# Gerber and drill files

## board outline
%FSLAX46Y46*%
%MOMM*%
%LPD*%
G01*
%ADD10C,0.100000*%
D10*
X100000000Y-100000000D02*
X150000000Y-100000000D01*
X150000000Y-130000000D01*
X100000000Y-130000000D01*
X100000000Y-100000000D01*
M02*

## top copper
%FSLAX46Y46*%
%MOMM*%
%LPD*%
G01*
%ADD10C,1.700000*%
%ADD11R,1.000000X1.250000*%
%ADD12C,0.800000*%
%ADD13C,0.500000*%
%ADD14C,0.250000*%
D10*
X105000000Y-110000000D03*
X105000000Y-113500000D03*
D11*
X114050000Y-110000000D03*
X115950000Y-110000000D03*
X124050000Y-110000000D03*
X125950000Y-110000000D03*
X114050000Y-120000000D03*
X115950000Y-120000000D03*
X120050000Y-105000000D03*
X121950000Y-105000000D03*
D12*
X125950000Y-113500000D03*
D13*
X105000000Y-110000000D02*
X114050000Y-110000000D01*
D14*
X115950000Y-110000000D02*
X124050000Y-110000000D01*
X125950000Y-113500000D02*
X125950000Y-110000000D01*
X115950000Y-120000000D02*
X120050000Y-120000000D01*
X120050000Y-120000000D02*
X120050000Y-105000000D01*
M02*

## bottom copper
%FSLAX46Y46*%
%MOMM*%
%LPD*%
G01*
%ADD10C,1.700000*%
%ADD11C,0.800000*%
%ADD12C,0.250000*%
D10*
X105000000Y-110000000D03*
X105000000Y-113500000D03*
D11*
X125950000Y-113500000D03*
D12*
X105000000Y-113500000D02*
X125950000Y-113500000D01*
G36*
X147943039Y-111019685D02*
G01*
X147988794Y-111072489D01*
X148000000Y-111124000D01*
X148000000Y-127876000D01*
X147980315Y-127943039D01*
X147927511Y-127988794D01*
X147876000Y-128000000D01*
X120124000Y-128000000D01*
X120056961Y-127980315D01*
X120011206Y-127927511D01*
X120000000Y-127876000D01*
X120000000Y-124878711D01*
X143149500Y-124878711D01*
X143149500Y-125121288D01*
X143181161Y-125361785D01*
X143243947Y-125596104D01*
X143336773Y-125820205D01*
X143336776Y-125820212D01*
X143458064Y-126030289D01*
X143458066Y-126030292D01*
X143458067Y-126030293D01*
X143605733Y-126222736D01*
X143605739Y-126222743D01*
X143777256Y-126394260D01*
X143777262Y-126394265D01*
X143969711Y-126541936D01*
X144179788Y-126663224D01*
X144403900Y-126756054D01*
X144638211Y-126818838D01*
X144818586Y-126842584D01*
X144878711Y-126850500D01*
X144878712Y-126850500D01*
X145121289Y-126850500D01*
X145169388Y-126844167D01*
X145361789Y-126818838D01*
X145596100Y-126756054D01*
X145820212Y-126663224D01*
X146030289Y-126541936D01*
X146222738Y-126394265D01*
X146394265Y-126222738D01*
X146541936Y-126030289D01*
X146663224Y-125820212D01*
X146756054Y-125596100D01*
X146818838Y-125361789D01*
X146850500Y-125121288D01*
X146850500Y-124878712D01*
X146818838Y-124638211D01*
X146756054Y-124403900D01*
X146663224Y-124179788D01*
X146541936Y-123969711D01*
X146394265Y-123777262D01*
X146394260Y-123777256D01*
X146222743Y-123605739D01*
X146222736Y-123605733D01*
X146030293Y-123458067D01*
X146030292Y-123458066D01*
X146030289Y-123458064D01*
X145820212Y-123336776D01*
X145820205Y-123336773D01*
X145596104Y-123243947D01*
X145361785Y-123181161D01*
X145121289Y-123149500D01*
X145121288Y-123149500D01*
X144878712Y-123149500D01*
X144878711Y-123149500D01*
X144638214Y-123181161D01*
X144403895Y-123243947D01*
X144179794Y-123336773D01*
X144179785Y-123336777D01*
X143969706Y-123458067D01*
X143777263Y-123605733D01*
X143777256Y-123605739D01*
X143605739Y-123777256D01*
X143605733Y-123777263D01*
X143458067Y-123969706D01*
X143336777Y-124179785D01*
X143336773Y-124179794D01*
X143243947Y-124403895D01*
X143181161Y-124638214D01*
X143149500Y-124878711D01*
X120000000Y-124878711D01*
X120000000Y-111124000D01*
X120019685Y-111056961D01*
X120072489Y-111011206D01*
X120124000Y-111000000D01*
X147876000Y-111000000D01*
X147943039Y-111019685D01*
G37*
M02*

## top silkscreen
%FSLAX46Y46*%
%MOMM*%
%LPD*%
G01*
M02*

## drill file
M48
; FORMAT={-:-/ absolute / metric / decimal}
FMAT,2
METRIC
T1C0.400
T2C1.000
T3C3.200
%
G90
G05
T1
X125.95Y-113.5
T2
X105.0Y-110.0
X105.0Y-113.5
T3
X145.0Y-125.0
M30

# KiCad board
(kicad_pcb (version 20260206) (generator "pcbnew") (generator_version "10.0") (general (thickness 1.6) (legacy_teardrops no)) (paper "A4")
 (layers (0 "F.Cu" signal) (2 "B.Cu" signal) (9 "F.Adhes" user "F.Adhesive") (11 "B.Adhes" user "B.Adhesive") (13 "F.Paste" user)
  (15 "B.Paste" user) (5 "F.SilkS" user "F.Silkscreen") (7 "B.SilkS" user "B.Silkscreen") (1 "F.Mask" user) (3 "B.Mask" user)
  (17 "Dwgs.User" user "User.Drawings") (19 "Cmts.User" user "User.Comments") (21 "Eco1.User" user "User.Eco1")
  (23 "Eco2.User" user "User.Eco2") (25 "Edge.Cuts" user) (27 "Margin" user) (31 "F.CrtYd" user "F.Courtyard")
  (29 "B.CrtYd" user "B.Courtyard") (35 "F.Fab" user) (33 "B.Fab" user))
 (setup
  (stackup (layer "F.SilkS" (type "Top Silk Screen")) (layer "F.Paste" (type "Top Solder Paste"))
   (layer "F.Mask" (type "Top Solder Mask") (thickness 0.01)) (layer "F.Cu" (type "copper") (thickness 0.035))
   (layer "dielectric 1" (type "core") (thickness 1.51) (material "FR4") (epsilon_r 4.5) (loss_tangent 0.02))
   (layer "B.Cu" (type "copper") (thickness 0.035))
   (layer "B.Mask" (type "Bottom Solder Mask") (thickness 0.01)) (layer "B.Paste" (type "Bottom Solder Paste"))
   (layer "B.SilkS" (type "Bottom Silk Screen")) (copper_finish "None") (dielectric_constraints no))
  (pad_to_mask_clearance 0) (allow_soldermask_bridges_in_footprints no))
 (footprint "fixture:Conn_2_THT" (layer "F.Cu") (at 105 110)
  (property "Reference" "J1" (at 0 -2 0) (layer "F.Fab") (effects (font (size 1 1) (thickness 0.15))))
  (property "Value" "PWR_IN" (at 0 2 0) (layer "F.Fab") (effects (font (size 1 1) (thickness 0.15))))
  (pad "1" thru_hole circle (at 0 0) (size 1.7 1.7) (drill 1) (layers "*.Cu" "*.Mask") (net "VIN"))
  (pad "2" thru_hole circle (at 0 3.5) (size 1.7 1.7) (drill 1) (layers "*.Cu" "*.Mask") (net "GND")))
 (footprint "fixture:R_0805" (layer "F.Cu") (at 115 110)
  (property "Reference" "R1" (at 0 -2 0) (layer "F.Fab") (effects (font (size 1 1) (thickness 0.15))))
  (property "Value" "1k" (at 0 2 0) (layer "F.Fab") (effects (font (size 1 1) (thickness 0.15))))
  (pad "1" smd rect (at -0.95 0) (size 1 1.25) (layers "F.Cu" "F.Paste" "F.Mask") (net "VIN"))
  (pad "2" smd rect (at 0.95 0) (size 1 1.25) (layers "F.Cu" "F.Paste" "F.Mask") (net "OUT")))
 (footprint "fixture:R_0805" (layer "F.Cu") (at 125 110)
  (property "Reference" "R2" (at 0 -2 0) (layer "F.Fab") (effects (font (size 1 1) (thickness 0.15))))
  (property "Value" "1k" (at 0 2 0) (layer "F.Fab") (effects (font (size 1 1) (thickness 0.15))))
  (pad "1" smd rect (at -0.95 0) (size 1 1.25) (layers "F.Cu" "F.Paste" "F.Mask") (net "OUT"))
  (pad "2" smd rect (at 0.95 0) (size 1 1.25) (layers "F.Cu" "F.Paste" "F.Mask") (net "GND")))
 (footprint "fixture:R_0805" (layer "F.Cu") (at 115 120)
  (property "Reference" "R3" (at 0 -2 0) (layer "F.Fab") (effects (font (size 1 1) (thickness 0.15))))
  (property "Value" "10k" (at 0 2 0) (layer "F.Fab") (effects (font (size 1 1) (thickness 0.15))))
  (pad "1" smd rect (at -0.95 0) (size 1 1.25) (layers "F.Cu" "F.Paste" "F.Mask") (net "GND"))
  (pad "2" smd rect (at 0.95 0) (size 1 1.25) (layers "F.Cu" "F.Paste" "F.Mask") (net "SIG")))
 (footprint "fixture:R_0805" (layer "F.Cu") (at 121 105)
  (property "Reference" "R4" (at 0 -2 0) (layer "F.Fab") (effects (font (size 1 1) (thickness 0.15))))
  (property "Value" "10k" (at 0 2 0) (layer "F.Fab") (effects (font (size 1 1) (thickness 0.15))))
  (pad "1" smd rect (at -0.95 0) (size 1 1.25) (layers "F.Cu" "F.Paste" "F.Mask") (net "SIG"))
  (pad "2" smd rect (at 0.95 0) (size 1 1.25) (layers "F.Cu" "F.Paste" "F.Mask") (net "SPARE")))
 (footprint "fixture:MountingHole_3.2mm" (layer "F.Cu") (at 145 125)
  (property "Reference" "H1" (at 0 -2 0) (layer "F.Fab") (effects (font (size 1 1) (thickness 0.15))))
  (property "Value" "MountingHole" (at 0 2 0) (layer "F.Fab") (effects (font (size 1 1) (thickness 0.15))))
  (pad "" np_thru_hole circle (at 0 0) (size 3.2 3.2) (drill 3.2) (layers "*.Cu" "*.Mask")))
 (gr_rect (start 100 100) (end 150 130) (stroke (width 0.1) (type solid)) (fill no) (layer "Edge.Cuts"))
 (segment (start 105 110) (end 114.05 110) (width 0.5) (layer "F.Cu") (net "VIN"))
 (segment (start 115.95 110) (end 124.05 110) (width 0.25) (layer "F.Cu") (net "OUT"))
 (segment (start 105 113.5) (end 125.95 113.5) (width 0.25) (layer "B.Cu") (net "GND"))
 (segment (start 125.95 113.5) (end 125.95 110) (width 0.25) (layer "F.Cu") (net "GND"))
 (segment (start 115.95 120) (end 120.05 120) (width 0.25) (layer "F.Cu") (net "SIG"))
 (segment (start 120.05 120) (end 120.05 105) (width 0.25) (layer "F.Cu") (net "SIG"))
 (via (at 125.95 113.5) (size 0.8) (drill 0.4) (layers "F.Cu" "B.Cu") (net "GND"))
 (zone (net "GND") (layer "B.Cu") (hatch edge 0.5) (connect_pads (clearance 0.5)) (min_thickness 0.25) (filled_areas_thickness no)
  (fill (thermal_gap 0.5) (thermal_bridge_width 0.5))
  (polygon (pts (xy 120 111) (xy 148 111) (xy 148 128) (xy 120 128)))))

